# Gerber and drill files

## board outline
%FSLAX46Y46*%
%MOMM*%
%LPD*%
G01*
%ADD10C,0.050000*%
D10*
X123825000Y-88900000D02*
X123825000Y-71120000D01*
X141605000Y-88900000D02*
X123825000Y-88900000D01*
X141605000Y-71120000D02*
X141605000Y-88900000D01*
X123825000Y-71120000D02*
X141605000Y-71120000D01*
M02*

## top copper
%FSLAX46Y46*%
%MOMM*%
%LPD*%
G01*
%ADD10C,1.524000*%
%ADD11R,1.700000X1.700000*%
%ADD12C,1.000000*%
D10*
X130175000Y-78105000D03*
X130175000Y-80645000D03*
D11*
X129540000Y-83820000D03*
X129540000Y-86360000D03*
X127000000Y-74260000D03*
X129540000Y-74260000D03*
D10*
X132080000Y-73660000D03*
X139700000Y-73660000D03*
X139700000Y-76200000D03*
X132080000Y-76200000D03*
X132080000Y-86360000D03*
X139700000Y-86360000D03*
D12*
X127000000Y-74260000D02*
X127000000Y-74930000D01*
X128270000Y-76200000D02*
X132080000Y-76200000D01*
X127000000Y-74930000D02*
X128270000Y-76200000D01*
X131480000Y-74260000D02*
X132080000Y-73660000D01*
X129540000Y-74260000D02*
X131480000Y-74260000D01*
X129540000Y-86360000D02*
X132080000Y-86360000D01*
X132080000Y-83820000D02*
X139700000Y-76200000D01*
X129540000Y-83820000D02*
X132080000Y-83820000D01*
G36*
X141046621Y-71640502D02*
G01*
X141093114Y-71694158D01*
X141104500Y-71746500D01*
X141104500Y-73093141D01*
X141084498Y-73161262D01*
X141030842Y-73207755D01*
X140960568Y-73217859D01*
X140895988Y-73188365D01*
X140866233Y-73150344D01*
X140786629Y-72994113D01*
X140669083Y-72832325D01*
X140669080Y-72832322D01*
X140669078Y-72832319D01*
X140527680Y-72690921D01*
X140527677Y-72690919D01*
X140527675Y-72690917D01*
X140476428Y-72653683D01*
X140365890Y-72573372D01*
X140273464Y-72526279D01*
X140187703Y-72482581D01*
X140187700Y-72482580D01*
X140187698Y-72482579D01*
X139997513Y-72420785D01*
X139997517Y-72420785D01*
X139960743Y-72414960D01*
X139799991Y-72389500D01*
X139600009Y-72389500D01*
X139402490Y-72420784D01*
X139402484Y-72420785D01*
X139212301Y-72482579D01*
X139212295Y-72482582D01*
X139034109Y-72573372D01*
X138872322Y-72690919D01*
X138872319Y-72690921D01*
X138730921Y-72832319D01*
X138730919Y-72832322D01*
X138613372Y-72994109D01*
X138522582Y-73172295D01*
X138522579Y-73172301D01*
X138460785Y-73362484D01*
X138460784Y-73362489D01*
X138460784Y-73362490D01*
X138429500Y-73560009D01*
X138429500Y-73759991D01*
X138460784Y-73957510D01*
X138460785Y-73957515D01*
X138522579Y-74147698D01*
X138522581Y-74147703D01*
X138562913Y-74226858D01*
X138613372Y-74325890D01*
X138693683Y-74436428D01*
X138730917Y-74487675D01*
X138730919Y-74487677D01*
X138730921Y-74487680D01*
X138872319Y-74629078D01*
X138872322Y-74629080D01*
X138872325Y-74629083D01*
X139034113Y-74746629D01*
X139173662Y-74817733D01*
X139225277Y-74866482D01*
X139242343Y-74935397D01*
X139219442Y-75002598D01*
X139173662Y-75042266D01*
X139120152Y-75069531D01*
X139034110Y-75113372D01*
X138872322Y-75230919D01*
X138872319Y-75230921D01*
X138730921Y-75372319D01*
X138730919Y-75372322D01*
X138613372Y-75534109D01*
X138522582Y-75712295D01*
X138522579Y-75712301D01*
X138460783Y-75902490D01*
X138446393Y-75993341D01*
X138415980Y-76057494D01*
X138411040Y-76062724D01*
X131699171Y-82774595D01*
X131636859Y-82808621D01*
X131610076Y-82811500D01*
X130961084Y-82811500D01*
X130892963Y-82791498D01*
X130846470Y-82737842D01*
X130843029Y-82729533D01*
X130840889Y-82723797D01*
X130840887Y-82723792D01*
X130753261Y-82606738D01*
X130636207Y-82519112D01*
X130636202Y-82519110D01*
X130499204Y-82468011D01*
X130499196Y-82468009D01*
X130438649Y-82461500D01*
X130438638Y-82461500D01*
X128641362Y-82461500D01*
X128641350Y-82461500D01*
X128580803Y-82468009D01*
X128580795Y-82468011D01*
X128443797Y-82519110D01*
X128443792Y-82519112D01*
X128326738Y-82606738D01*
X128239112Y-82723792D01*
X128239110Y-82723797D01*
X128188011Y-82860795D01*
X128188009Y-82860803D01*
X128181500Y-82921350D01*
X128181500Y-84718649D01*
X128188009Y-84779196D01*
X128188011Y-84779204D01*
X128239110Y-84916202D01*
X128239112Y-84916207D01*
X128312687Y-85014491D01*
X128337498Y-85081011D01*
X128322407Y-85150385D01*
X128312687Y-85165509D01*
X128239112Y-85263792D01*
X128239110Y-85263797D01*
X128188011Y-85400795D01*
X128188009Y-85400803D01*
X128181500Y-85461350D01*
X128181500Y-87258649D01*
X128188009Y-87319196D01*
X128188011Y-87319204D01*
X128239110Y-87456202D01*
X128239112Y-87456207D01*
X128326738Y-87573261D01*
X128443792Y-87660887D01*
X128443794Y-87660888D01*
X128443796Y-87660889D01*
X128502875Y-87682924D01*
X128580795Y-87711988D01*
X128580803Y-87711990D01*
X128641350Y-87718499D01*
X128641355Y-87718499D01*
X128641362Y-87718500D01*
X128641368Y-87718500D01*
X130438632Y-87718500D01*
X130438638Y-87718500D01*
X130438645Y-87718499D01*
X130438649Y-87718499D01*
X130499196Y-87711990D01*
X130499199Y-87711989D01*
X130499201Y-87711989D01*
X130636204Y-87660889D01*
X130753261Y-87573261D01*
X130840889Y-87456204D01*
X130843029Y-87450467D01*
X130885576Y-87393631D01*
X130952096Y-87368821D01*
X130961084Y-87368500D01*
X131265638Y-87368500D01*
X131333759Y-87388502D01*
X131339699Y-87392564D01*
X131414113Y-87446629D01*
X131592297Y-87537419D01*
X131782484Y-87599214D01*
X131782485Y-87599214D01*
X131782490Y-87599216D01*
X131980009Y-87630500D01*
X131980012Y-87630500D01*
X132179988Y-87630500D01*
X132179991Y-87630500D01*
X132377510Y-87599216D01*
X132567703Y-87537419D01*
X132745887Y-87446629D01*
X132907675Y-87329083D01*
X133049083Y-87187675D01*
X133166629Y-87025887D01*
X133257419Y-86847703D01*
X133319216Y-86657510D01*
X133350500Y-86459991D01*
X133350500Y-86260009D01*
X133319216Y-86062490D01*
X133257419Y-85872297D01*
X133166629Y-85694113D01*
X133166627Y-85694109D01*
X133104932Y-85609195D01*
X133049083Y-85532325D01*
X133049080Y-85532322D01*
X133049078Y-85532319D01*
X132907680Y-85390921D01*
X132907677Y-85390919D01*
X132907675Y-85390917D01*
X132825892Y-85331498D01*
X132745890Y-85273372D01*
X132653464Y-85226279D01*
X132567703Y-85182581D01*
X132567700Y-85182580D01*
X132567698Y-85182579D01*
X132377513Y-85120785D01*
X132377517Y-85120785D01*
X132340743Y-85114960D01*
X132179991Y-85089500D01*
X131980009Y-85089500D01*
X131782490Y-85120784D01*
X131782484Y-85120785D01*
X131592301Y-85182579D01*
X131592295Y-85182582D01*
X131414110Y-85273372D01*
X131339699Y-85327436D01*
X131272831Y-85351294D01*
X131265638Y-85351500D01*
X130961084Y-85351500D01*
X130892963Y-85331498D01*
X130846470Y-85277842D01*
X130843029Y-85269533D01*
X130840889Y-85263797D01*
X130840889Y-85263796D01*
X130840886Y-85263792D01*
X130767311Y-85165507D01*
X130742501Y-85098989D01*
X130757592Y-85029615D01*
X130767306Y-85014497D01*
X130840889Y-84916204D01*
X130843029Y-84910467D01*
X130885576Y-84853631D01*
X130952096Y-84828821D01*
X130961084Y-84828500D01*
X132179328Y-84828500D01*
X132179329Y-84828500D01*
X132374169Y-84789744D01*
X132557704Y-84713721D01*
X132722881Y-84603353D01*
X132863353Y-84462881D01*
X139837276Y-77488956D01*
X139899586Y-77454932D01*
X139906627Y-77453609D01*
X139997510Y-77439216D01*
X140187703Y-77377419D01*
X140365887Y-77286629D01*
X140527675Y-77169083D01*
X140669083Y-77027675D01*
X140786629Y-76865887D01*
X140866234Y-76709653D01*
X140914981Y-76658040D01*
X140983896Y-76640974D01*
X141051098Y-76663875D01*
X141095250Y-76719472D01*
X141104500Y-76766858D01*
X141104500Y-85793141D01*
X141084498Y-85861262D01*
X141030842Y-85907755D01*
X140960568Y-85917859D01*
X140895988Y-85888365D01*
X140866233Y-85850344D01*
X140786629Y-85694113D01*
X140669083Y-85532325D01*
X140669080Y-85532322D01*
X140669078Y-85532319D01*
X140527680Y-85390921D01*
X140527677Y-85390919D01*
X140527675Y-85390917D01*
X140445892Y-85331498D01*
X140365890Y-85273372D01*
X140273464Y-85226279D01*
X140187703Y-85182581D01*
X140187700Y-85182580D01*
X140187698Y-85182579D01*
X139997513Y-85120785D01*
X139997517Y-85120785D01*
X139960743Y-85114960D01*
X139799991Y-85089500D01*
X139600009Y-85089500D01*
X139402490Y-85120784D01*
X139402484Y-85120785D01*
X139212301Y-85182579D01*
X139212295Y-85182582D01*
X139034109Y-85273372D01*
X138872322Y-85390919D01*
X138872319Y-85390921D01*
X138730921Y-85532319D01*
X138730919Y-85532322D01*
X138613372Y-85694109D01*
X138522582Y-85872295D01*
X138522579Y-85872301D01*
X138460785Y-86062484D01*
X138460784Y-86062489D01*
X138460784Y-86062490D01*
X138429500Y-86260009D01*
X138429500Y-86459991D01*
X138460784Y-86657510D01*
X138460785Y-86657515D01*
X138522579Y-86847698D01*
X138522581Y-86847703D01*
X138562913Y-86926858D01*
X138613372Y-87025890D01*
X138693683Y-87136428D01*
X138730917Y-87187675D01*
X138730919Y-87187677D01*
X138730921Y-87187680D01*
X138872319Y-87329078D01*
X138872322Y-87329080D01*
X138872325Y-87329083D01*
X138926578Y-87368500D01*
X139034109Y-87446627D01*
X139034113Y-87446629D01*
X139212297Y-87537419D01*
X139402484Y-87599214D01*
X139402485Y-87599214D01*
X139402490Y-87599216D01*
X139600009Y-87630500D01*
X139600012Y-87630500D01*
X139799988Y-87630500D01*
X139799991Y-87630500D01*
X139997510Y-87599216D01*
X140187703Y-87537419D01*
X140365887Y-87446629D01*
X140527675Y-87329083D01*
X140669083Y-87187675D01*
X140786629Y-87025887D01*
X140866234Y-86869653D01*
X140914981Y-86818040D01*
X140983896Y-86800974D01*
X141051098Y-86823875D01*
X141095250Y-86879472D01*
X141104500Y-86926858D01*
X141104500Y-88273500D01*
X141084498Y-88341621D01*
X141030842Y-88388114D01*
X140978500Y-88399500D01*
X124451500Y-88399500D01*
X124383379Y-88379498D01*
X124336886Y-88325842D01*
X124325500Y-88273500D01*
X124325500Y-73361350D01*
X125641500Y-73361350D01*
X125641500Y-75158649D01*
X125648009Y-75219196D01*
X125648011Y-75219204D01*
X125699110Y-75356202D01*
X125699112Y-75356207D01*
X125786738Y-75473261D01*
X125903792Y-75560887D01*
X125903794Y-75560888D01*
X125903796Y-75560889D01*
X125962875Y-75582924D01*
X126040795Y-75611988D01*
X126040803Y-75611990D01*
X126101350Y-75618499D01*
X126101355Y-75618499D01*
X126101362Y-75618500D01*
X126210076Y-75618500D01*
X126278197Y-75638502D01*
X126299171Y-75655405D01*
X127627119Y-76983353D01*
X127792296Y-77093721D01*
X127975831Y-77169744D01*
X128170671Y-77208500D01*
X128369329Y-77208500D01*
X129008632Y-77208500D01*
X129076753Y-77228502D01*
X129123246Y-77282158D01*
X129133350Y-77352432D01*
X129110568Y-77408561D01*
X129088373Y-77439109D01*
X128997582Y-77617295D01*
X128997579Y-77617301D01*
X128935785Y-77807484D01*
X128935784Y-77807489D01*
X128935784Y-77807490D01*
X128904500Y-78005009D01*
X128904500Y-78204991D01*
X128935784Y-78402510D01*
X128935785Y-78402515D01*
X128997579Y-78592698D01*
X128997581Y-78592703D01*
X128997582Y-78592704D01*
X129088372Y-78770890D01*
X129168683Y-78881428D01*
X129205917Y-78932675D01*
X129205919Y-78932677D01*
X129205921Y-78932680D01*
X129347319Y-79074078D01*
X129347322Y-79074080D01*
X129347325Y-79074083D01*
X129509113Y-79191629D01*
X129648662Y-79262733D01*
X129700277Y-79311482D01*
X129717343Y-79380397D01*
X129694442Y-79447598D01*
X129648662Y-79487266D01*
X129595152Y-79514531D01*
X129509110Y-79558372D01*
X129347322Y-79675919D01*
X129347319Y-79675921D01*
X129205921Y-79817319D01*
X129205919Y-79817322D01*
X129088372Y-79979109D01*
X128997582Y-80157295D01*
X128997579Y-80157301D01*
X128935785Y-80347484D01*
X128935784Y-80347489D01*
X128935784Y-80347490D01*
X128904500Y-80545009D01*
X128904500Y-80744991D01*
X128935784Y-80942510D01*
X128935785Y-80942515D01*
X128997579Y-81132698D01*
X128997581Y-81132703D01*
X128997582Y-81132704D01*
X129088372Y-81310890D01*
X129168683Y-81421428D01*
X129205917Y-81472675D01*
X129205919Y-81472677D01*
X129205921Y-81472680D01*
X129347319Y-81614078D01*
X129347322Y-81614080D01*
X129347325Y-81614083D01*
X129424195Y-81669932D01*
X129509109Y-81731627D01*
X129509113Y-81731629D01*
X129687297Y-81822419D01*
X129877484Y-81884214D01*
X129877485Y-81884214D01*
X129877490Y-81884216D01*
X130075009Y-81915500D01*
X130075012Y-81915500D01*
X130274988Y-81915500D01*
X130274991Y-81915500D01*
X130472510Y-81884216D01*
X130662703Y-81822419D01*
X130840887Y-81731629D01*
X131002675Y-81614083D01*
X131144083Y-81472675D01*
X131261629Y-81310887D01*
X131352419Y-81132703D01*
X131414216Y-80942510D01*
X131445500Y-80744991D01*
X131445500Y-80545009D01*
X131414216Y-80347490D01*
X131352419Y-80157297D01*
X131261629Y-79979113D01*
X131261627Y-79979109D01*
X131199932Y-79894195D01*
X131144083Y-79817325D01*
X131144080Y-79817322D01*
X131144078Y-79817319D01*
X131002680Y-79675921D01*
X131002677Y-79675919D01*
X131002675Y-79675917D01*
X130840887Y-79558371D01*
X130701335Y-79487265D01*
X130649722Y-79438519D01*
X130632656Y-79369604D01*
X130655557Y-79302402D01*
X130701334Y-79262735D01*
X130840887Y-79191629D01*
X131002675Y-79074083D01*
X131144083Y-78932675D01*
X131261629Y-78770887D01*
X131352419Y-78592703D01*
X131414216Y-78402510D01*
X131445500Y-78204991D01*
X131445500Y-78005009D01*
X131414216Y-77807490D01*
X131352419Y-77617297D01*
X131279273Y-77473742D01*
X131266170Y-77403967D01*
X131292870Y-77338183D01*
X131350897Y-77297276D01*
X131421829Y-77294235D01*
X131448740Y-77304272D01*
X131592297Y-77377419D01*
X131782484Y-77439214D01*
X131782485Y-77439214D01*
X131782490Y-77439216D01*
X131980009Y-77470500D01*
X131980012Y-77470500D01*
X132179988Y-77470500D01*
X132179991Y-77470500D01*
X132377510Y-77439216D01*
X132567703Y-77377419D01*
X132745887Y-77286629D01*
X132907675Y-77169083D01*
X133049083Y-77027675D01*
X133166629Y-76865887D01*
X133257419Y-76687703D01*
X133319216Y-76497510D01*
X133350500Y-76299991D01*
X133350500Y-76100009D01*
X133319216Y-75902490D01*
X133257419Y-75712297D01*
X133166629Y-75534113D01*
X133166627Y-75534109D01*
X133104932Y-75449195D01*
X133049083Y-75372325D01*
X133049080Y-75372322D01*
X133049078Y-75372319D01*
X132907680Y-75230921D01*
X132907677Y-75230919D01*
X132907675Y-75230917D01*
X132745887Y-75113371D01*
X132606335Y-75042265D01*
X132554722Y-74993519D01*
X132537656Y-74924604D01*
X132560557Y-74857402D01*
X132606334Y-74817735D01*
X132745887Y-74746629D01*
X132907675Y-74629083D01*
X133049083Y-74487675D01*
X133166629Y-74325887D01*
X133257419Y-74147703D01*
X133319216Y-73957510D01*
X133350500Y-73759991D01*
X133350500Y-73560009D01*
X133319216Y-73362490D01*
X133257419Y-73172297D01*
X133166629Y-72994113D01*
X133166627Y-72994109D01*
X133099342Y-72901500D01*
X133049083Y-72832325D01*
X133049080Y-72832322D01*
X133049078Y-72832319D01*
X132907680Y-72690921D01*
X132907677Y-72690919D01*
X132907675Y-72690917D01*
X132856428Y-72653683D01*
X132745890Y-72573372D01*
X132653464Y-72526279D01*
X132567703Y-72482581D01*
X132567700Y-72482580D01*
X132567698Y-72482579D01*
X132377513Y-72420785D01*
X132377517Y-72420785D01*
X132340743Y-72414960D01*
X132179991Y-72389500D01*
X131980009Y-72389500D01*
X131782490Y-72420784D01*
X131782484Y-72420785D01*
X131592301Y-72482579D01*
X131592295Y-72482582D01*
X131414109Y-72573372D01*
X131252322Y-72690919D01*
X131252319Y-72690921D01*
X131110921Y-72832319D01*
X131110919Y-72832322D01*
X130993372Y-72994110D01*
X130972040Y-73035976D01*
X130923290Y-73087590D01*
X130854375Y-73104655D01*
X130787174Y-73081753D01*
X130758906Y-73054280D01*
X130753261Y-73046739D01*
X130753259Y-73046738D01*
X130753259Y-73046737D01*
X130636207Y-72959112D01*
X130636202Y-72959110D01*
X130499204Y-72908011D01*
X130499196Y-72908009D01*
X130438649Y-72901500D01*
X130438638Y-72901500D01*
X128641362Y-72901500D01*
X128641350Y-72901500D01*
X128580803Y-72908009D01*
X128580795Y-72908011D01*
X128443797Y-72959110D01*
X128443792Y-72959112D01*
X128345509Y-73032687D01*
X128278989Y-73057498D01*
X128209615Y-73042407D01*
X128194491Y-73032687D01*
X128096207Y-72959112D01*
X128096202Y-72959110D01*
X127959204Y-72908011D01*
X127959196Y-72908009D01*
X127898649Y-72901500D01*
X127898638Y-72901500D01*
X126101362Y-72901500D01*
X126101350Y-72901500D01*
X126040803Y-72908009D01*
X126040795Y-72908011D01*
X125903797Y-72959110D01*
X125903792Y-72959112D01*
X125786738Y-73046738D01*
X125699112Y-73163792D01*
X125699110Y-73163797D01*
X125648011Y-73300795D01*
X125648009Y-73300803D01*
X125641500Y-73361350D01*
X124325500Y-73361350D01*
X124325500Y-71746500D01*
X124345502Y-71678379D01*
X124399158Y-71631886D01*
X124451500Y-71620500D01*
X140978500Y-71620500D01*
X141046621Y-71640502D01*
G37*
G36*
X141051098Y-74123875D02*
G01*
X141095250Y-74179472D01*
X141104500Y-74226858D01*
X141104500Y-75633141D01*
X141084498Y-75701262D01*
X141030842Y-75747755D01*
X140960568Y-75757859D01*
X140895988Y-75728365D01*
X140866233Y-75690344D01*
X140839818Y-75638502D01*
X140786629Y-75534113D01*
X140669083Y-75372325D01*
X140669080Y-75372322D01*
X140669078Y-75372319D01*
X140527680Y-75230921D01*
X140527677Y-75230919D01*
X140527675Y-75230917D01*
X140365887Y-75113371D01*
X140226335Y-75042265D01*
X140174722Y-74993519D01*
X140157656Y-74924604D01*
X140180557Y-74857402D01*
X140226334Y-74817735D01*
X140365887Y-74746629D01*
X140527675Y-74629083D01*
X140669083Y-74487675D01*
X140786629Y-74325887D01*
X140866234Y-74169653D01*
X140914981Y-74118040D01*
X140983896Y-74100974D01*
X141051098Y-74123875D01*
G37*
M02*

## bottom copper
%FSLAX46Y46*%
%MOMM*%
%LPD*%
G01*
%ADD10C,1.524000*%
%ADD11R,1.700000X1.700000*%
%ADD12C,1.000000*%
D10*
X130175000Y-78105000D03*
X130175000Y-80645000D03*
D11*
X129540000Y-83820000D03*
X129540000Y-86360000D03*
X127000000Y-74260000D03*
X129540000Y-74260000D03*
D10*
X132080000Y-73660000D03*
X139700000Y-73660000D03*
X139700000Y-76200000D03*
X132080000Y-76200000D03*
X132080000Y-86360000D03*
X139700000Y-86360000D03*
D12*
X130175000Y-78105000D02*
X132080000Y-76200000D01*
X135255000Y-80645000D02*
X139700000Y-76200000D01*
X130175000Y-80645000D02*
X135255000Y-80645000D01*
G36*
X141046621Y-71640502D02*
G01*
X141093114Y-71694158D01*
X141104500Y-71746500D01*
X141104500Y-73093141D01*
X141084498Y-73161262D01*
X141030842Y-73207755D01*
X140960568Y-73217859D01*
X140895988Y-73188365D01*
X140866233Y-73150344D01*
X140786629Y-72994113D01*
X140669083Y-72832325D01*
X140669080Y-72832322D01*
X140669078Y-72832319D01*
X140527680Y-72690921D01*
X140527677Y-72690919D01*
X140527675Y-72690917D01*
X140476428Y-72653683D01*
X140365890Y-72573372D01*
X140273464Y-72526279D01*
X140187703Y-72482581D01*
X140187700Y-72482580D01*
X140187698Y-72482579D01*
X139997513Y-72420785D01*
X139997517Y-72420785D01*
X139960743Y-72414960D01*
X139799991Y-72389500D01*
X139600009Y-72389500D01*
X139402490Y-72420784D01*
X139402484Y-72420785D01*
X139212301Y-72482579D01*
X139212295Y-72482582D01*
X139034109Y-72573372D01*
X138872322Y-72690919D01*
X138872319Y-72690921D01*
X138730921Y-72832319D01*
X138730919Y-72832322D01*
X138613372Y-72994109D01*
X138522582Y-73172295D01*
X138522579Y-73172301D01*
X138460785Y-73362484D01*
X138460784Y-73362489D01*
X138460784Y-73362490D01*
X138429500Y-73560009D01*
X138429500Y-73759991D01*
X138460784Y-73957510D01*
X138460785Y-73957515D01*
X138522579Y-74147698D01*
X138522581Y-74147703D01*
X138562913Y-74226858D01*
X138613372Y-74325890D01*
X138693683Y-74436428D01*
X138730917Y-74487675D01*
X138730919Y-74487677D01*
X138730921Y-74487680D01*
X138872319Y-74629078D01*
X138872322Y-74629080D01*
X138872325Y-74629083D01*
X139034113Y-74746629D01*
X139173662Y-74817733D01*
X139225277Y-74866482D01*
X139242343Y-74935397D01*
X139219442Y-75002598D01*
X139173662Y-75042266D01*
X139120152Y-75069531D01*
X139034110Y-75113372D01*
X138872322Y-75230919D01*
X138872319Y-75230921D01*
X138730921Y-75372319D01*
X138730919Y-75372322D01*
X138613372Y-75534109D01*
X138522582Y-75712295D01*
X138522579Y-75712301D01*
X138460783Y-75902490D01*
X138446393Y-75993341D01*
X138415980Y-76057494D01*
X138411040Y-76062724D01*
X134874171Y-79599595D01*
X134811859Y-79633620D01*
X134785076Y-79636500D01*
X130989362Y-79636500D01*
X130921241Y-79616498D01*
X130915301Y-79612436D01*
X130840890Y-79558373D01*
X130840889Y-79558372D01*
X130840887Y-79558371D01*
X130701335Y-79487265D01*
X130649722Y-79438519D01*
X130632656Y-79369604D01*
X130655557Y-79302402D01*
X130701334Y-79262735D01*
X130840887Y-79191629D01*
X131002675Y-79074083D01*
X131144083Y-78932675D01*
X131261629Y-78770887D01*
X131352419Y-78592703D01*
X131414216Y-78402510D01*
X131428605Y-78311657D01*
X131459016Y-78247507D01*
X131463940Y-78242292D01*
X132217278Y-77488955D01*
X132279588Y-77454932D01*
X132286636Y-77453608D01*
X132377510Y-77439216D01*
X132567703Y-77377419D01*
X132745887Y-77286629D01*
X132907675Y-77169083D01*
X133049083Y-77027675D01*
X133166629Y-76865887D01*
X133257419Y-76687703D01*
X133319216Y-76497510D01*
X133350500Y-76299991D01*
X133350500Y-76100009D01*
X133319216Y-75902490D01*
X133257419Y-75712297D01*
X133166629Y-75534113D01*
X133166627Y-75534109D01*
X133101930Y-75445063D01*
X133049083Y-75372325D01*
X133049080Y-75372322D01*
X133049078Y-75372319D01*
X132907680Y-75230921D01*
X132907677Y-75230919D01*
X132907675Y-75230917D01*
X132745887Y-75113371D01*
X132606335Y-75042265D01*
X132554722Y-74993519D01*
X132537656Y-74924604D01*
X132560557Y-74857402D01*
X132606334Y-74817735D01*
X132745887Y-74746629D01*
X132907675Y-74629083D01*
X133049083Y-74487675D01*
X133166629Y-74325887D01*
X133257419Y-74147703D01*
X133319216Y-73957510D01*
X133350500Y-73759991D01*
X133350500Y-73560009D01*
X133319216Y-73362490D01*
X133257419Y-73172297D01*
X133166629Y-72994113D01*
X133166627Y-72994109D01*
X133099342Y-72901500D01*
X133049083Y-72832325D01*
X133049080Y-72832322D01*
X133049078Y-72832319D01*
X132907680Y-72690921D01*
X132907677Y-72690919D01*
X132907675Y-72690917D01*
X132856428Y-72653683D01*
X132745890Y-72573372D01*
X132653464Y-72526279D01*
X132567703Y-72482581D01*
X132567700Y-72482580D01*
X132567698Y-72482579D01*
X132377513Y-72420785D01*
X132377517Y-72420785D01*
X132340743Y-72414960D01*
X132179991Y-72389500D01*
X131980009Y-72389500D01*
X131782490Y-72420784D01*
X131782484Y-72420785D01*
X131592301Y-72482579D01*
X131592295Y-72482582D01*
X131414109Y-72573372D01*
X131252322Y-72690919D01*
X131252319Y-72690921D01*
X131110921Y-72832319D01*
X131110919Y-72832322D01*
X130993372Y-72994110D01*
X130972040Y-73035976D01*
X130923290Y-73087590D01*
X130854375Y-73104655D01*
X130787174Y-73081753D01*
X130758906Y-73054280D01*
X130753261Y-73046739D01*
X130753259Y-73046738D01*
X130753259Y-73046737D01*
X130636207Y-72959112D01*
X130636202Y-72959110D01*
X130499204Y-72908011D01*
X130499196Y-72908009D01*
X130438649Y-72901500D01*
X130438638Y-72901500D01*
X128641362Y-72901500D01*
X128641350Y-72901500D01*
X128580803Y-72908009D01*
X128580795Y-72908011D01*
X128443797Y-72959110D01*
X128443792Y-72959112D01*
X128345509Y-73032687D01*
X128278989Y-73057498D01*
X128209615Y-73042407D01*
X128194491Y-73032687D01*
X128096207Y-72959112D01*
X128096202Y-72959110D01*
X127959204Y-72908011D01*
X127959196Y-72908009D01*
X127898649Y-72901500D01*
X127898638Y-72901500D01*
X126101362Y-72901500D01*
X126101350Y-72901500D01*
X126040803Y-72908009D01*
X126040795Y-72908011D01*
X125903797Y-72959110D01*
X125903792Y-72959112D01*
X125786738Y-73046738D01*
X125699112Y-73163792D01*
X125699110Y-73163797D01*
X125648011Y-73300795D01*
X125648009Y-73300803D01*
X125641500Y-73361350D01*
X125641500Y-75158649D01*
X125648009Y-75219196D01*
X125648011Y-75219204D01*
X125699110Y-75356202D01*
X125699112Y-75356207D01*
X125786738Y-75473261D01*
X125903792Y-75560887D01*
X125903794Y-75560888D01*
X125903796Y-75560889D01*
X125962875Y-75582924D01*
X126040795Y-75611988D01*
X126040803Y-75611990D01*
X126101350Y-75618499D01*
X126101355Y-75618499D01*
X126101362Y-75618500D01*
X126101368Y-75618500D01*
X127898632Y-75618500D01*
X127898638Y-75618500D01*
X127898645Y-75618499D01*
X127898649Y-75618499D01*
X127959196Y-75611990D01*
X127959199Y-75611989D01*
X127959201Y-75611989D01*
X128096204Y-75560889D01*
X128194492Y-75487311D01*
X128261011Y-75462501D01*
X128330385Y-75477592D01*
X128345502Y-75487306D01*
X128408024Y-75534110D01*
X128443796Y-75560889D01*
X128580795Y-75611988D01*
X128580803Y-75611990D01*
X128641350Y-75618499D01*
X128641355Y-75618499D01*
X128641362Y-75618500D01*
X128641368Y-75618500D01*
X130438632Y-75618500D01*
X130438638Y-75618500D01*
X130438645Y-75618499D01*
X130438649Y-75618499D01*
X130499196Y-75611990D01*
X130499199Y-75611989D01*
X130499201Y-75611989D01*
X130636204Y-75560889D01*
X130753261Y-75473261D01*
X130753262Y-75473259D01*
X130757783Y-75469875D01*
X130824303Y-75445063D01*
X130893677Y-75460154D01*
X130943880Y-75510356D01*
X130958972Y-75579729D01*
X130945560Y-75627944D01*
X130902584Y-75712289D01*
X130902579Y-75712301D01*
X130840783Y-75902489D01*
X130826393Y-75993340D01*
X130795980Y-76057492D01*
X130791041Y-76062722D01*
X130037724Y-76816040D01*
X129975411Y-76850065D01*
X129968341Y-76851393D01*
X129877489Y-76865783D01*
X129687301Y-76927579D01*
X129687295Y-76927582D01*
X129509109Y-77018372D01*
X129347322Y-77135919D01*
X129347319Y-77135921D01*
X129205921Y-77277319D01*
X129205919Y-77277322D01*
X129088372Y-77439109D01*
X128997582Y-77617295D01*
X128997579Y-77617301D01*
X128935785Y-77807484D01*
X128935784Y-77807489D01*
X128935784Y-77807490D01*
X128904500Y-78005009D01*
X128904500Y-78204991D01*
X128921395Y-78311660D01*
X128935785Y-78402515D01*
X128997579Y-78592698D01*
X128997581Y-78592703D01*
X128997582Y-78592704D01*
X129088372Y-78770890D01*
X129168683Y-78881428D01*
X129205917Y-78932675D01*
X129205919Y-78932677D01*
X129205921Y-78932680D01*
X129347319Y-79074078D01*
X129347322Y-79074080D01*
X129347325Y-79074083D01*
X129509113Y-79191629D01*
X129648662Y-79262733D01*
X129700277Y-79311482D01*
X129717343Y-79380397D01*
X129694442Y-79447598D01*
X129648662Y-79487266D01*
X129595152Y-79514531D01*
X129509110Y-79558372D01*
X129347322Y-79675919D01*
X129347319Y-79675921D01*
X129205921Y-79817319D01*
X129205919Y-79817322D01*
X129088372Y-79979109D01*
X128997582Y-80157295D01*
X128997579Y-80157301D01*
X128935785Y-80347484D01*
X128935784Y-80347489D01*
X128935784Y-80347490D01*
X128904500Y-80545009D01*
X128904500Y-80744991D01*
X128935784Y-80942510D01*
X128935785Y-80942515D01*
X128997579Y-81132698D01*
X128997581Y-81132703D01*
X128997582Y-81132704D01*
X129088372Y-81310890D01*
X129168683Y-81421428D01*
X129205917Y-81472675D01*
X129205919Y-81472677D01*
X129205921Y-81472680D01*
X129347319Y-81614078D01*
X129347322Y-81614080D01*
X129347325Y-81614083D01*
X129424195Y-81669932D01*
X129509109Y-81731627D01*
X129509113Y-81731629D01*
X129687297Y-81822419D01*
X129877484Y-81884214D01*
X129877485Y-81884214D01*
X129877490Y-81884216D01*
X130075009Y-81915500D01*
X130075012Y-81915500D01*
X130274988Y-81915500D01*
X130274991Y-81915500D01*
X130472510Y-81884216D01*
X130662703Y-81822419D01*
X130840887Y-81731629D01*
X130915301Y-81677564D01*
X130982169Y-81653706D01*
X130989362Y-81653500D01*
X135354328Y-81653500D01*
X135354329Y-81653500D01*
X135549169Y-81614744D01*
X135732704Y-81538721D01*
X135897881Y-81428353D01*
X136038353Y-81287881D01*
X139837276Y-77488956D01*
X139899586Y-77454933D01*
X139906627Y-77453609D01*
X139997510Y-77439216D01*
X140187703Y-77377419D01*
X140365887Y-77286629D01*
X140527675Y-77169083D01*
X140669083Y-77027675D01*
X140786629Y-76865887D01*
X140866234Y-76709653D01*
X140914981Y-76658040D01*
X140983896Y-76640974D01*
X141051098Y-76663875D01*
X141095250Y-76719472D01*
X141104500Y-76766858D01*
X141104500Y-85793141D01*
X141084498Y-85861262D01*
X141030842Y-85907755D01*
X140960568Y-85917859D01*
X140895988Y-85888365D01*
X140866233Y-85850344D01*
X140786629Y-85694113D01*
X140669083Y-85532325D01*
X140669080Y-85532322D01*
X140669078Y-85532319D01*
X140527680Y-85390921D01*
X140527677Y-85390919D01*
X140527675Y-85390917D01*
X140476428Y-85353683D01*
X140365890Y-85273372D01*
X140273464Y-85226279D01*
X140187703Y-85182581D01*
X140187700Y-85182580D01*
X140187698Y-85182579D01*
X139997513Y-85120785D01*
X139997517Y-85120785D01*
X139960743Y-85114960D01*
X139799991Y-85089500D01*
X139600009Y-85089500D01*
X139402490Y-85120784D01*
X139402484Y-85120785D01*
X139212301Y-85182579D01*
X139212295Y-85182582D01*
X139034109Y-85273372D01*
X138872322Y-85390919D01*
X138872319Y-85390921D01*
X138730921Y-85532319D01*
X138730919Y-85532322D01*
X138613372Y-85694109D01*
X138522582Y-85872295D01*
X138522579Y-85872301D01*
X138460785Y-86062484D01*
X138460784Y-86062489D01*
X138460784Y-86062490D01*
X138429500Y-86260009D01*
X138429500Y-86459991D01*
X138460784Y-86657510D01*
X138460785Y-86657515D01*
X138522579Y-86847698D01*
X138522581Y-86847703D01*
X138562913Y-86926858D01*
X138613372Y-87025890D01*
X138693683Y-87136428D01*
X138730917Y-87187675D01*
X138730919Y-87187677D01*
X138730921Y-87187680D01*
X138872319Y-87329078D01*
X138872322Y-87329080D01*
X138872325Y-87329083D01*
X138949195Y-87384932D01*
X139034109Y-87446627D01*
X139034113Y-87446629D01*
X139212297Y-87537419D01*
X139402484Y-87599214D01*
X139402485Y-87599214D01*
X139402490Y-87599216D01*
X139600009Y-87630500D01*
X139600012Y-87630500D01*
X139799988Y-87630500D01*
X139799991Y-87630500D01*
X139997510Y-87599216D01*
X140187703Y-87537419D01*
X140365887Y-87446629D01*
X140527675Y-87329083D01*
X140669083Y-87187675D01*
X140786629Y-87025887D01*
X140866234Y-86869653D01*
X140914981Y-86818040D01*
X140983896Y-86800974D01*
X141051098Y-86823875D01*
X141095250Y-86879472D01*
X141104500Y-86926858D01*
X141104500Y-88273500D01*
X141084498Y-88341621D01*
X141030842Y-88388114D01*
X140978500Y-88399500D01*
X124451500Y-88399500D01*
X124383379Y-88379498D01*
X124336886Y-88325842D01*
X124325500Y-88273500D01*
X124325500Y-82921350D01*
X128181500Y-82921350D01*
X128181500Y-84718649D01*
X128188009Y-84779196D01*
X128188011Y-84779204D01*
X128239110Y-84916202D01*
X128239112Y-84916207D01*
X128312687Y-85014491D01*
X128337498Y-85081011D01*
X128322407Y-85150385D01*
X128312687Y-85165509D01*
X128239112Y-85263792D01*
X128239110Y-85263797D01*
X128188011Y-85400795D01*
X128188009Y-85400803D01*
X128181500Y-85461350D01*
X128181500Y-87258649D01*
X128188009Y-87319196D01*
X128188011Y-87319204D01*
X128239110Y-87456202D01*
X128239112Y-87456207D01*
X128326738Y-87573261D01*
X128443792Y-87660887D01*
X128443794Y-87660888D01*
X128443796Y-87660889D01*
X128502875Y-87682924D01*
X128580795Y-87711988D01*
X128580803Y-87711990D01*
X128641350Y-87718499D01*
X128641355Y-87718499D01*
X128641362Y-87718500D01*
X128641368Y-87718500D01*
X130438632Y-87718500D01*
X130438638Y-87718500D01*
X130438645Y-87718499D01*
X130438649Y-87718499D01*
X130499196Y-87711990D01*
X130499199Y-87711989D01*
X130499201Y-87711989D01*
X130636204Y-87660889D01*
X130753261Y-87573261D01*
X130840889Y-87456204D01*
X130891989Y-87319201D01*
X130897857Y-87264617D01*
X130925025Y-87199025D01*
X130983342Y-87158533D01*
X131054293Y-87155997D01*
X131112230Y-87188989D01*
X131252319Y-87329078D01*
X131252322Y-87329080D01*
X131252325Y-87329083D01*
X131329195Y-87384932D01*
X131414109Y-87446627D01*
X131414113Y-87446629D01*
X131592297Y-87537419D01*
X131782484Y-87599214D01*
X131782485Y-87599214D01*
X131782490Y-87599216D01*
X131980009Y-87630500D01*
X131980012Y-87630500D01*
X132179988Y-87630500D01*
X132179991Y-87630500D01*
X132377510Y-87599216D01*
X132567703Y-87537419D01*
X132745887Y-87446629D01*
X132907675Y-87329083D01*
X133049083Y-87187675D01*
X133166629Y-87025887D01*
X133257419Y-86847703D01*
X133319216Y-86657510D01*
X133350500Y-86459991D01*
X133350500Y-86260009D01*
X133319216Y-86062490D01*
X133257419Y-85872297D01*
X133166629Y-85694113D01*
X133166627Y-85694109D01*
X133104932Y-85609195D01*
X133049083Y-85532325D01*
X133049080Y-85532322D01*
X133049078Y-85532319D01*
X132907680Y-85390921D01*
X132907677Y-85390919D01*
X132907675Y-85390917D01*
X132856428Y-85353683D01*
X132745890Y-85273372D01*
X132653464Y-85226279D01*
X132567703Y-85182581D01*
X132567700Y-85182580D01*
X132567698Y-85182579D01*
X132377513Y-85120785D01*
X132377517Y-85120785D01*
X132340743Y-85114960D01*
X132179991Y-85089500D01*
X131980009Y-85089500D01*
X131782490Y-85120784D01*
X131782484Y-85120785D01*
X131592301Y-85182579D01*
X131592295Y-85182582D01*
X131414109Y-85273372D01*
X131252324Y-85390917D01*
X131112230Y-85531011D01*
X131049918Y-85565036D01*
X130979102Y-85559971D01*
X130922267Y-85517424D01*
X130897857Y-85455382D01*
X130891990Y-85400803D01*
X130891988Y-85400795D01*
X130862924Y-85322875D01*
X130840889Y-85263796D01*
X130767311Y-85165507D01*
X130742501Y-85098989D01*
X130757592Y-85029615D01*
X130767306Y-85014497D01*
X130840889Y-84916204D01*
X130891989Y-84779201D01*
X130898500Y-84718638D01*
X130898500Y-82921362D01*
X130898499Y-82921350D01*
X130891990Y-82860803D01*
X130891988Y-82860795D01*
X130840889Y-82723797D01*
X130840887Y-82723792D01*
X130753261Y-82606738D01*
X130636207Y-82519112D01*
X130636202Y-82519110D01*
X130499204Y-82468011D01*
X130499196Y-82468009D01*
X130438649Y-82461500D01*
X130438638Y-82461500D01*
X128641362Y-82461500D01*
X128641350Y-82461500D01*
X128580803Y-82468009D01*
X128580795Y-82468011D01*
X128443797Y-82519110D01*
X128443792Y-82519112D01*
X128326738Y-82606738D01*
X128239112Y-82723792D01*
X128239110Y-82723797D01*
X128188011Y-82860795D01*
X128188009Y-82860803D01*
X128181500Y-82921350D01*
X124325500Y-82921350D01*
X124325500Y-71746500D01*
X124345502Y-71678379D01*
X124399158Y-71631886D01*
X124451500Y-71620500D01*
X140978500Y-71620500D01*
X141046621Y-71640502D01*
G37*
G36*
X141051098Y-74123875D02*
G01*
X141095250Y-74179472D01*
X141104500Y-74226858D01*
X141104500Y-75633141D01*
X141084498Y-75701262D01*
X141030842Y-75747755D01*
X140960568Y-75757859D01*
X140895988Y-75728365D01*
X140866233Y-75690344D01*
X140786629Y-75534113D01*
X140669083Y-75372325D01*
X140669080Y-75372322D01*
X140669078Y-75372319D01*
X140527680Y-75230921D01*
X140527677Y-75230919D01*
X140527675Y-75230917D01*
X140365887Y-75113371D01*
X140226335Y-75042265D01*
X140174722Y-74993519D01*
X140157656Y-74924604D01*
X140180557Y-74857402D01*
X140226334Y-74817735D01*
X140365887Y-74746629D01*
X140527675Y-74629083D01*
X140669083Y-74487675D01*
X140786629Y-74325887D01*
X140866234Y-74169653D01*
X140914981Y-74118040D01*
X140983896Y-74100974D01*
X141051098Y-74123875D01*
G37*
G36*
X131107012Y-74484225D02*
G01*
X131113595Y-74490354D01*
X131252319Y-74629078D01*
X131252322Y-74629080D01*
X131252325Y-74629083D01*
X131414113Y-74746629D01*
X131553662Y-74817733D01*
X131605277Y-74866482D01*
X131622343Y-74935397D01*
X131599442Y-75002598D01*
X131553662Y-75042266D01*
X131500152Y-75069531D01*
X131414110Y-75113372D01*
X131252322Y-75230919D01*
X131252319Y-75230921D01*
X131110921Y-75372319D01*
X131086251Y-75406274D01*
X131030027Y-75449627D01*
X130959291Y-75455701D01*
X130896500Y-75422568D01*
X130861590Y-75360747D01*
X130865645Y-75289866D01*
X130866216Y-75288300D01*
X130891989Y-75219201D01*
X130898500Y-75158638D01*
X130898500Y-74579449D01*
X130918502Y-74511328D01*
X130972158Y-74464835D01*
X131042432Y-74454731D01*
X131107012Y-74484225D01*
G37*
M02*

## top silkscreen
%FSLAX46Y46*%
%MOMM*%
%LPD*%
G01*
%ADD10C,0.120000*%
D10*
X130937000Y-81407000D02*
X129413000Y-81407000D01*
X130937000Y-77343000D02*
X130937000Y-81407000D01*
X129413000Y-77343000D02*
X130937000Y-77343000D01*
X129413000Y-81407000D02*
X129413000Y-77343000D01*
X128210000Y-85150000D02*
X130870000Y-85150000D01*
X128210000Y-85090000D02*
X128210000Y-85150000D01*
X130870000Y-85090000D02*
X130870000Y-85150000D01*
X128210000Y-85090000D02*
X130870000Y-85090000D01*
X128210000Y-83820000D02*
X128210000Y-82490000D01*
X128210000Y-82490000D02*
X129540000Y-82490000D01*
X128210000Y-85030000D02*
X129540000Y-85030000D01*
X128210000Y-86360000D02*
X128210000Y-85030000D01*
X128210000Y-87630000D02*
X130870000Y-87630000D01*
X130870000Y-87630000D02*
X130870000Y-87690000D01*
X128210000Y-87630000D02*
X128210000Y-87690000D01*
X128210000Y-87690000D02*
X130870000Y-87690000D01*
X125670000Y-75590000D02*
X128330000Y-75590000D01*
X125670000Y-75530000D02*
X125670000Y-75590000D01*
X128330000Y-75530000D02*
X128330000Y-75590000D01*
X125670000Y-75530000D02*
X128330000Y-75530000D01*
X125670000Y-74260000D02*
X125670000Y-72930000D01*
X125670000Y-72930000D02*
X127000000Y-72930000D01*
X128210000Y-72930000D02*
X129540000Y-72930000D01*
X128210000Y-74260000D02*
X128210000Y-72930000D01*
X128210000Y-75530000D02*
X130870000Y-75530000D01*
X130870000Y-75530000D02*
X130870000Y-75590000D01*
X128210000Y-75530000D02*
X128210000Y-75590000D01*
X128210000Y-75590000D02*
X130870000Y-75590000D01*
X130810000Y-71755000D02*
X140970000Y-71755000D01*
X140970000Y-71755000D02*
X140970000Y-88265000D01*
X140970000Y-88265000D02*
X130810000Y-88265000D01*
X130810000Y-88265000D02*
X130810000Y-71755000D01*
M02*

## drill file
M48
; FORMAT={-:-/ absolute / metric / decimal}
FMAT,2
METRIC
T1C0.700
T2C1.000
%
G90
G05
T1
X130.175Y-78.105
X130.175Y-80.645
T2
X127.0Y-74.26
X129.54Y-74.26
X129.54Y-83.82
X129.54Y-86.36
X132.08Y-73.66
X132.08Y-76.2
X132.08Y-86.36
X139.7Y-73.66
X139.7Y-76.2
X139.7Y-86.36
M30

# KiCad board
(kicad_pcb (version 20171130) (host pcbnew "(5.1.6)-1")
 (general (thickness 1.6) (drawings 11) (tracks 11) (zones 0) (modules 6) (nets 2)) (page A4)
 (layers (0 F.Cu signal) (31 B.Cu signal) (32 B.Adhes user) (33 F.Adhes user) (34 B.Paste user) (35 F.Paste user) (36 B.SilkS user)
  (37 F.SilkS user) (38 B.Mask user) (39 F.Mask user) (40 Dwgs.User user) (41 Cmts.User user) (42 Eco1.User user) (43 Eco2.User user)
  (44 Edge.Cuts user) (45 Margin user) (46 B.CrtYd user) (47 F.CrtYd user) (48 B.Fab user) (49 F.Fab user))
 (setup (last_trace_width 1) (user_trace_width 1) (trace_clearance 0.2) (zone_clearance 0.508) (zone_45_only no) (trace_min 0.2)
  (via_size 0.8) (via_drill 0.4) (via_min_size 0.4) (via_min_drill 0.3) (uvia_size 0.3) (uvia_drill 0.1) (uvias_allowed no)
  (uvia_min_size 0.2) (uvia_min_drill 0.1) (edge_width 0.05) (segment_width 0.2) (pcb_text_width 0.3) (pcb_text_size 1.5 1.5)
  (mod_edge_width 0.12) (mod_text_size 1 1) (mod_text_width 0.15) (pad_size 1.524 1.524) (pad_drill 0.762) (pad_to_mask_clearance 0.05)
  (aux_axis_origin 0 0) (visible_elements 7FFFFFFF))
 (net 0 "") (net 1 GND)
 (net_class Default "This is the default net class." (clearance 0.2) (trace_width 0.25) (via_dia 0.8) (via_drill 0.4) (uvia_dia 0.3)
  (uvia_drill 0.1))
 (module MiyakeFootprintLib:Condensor (layer F.Cu) (at 130.175 80.645 90)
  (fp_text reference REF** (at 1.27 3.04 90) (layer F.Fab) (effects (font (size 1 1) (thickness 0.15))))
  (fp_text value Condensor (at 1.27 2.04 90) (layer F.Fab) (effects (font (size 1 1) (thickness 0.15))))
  (fp_line (start -0.762 0.762) (end -0.762 -0.762) (layer F.SilkS) (width 0.12))
  (fp_line (start 3.302 0.762) (end -0.762 0.762) (layer F.SilkS) (width 0.12))
  (fp_line (start 3.302 -0.762) (end 3.302 0.762) (layer F.SilkS) (width 0.12))
  (fp_line (start -0.762 -0.762) (end 3.302 -0.762) (layer F.SilkS) (width 0.12))
  (pad 2 thru_hole circle (at 2.54 0 90) (size 1.524 1.524) (drill 0.7) (layers *.Cu *.Mask))
  (pad 1 thru_hole circle (at 0 0 90) (size 1.524 1.524) (drill 0.7) (layers *.Cu *.Mask)))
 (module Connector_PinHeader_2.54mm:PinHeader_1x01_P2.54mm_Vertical (layer F.Cu) (at 129.54 83.82)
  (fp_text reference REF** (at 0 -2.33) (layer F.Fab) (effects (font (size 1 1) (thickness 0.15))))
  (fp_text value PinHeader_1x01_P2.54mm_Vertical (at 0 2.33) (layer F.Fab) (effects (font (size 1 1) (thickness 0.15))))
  (fp_line (start -1.33 1.33) (end 1.33 1.33) (layer F.SilkS) (width 0.12))
  (fp_line (start -1.33 1.27) (end -1.33 1.33) (layer F.SilkS) (width 0.12))
  (fp_line (start 1.33 1.27) (end 1.33 1.33) (layer F.SilkS) (width 0.12))
  (fp_line (start -1.33 1.27) (end 1.33 1.27) (layer F.SilkS) (width 0.12))
  (fp_line (start -1.33 0) (end -1.33 -1.33) (layer F.SilkS) (width 0.12))
  (fp_line (start -1.33 -1.33) (end 0 -1.33) (layer F.SilkS) (width 0.12))
  (pad 1 thru_hole rect (at 0 0) (size 1.7 1.7) (drill 1) (layers *.Cu *.Mask)))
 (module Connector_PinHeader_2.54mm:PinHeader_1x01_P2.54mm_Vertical (layer F.Cu) (at 129.54 86.36)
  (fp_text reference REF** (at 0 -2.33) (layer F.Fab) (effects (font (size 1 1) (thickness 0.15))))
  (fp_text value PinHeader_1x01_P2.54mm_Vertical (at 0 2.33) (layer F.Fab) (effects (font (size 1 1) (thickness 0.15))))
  (fp_line (start -1.33 -1.33) (end 0 -1.33) (layer F.SilkS) (width 0.12))
  (fp_line (start -1.33 0) (end -1.33 -1.33) (layer F.SilkS) (width 0.12))
  (fp_line (start -1.33 1.27) (end 1.33 1.27) (layer F.SilkS) (width 0.12))
  (fp_line (start 1.33 1.27) (end 1.33 1.33) (layer F.SilkS) (width 0.12))
  (fp_line (start -1.33 1.27) (end -1.33 1.33) (layer F.SilkS) (width 0.12))
  (fp_line (start -1.33 1.33) (end 1.33 1.33) (layer F.SilkS) (width 0.12))
  (pad 1 thru_hole rect (at 0 0) (size 1.7 1.7) (drill 1) (layers *.Cu *.Mask)))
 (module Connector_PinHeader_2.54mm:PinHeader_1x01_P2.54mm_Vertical (layer F.Cu) (at 127 74.26)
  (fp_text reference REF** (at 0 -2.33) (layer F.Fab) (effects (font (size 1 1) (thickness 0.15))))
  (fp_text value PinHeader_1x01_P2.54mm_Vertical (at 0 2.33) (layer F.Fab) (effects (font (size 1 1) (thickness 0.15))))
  (fp_line (start -1.33 1.33) (end 1.33 1.33) (layer F.SilkS) (width 0.12))
  (fp_line (start -1.33 1.27) (end -1.33 1.33) (layer F.SilkS) (width 0.12))
  (fp_line (start 1.33 1.27) (end 1.33 1.33) (layer F.SilkS) (width 0.12))
  (fp_line (start -1.33 1.27) (end 1.33 1.27) (layer F.SilkS) (width 0.12))
  (fp_line (start -1.33 0) (end -1.33 -1.33) (layer F.SilkS) (width 0.12))
  (fp_line (start -1.33 -1.33) (end 0 -1.33) (layer F.SilkS) (width 0.12))
  (pad 1 thru_hole rect (at 0 0) (size 1.7 1.7) (drill 1) (layers *.Cu *.Mask)))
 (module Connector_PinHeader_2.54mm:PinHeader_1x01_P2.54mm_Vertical (layer F.Cu) (at 129.54 74.26)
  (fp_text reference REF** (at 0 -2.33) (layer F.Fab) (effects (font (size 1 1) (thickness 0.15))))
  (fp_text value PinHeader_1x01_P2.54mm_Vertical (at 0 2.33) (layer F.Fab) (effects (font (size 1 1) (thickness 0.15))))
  (fp_line (start -1.33 -1.33) (end 0 -1.33) (layer F.SilkS) (width 0.12))
  (fp_line (start -1.33 0) (end -1.33 -1.33) (layer F.SilkS) (width 0.12))
  (fp_line (start -1.33 1.27) (end 1.33 1.27) (layer F.SilkS) (width 0.12))
  (fp_line (start 1.33 1.27) (end 1.33 1.33) (layer F.SilkS) (width 0.12))
  (fp_line (start -1.33 1.27) (end -1.33 1.33) (layer F.SilkS) (width 0.12))
  (fp_line (start -1.33 1.33) (end 1.33 1.33) (layer F.SilkS) (width 0.12))
  (pad 1 thru_hole rect (at 0 0) (size 1.7 1.7) (drill 1) (layers *.Cu *.Mask)))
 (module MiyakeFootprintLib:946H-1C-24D (layer F.Cu) (at 137.16 78.74)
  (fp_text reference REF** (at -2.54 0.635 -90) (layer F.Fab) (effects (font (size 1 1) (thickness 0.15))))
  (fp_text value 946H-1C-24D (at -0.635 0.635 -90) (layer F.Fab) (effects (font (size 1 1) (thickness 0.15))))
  (fp_line (start -6.35 -6.985) (end 3.81 -6.985) (layer F.SilkS) (width 0.12))
  (fp_line (start 3.81 -6.985) (end 3.81 9.525) (layer F.SilkS) (width 0.12))
  (fp_line (start 3.81 9.525) (end -6.35 9.525) (layer F.SilkS) (width 0.12))
  (fp_line (start -6.35 9.525) (end -6.35 -6.985) (layer F.SilkS) (width 0.12))
  (pad 1 thru_hole circle (at -5.08 -5.08) (size 1.524 1.524) (drill 1) (layers *.Cu *.Mask))
  (pad 2 thru_hole circle (at 2.54 -5.08) (size 1.524 1.524) (drill 1) (layers *.Cu *.Mask))
  (pad 3 thru_hole circle (at 2.54 -2.54) (size 1.524 1.524) (drill 1) (layers *.Cu *.Mask))
  (pad 4 thru_hole circle (at -5.08 -2.54) (size 1.524 1.524) (drill 1) (layers *.Cu *.Mask))
  (pad 5 thru_hole circle (at -5.08 7.62) (size 1.524 1.524) (drill 1) (layers *.Cu *.Mask))
  (pad 6 thru_hole circle (at 2.54 7.62) (size 1.524 1.524) (drill 1) (layers *.Cu *.Mask)))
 (gr_line (start 123.825 88.9) (end 123.825 71.12) (layer Edge.Cuts) (width 0.05))
 (gr_line (start 141.605 88.9) (end 123.825 88.9) (layer Edge.Cuts) (width 0.05))
 (gr_line (start 141.605 71.12) (end 141.605 88.9) (layer Edge.Cuts) (width 0.05))
 (gr_line (start 123.825 71.12) (end 141.605 71.12) (layer Edge.Cuts) (width 0.05))
 (segment (start 127 74.26) (end 127 74.93) (width 1) (layer F.Cu) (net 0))
 (segment (start 128.27 76.2) (end 132.08 76.2) (width 1) (layer F.Cu) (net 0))
 (segment (start 127 74.93) (end 128.27 76.2) (width 1) (layer F.Cu) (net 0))
 (segment (start 131.48 74.26) (end 132.08 73.66) (width 1) (layer F.Cu) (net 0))
 (segment (start 129.54 74.26) (end 131.48 74.26) (width 1) (layer F.Cu) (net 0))
 (segment (start 129.54 86.36) (end 132.08 86.36) (width 1) (layer F.Cu) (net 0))
 (segment (start 132.08 83.82) (end 139.7 76.2) (width 1) (layer F.Cu) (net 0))
 (segment (start 129.54 83.82) (end 132.08 83.82) (width 1) (layer F.Cu) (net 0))
 (segment (start 130.175 78.105) (end 132.08 76.2) (width 1) (layer B.Cu) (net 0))
 (segment (start 135.255 80.645) (end 139.7 76.2) (width 1) (layer B.Cu) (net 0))
 (segment (start 130.175 80.645) (end 135.255 80.645) (width 1) (layer B.Cu) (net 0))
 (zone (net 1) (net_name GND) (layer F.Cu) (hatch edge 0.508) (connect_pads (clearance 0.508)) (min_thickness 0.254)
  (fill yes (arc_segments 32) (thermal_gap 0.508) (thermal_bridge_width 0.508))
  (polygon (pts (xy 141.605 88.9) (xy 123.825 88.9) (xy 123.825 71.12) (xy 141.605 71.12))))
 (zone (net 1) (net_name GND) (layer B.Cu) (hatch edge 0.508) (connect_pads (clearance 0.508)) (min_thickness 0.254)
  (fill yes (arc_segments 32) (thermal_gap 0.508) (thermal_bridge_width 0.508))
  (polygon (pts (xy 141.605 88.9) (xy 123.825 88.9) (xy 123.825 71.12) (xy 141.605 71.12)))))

